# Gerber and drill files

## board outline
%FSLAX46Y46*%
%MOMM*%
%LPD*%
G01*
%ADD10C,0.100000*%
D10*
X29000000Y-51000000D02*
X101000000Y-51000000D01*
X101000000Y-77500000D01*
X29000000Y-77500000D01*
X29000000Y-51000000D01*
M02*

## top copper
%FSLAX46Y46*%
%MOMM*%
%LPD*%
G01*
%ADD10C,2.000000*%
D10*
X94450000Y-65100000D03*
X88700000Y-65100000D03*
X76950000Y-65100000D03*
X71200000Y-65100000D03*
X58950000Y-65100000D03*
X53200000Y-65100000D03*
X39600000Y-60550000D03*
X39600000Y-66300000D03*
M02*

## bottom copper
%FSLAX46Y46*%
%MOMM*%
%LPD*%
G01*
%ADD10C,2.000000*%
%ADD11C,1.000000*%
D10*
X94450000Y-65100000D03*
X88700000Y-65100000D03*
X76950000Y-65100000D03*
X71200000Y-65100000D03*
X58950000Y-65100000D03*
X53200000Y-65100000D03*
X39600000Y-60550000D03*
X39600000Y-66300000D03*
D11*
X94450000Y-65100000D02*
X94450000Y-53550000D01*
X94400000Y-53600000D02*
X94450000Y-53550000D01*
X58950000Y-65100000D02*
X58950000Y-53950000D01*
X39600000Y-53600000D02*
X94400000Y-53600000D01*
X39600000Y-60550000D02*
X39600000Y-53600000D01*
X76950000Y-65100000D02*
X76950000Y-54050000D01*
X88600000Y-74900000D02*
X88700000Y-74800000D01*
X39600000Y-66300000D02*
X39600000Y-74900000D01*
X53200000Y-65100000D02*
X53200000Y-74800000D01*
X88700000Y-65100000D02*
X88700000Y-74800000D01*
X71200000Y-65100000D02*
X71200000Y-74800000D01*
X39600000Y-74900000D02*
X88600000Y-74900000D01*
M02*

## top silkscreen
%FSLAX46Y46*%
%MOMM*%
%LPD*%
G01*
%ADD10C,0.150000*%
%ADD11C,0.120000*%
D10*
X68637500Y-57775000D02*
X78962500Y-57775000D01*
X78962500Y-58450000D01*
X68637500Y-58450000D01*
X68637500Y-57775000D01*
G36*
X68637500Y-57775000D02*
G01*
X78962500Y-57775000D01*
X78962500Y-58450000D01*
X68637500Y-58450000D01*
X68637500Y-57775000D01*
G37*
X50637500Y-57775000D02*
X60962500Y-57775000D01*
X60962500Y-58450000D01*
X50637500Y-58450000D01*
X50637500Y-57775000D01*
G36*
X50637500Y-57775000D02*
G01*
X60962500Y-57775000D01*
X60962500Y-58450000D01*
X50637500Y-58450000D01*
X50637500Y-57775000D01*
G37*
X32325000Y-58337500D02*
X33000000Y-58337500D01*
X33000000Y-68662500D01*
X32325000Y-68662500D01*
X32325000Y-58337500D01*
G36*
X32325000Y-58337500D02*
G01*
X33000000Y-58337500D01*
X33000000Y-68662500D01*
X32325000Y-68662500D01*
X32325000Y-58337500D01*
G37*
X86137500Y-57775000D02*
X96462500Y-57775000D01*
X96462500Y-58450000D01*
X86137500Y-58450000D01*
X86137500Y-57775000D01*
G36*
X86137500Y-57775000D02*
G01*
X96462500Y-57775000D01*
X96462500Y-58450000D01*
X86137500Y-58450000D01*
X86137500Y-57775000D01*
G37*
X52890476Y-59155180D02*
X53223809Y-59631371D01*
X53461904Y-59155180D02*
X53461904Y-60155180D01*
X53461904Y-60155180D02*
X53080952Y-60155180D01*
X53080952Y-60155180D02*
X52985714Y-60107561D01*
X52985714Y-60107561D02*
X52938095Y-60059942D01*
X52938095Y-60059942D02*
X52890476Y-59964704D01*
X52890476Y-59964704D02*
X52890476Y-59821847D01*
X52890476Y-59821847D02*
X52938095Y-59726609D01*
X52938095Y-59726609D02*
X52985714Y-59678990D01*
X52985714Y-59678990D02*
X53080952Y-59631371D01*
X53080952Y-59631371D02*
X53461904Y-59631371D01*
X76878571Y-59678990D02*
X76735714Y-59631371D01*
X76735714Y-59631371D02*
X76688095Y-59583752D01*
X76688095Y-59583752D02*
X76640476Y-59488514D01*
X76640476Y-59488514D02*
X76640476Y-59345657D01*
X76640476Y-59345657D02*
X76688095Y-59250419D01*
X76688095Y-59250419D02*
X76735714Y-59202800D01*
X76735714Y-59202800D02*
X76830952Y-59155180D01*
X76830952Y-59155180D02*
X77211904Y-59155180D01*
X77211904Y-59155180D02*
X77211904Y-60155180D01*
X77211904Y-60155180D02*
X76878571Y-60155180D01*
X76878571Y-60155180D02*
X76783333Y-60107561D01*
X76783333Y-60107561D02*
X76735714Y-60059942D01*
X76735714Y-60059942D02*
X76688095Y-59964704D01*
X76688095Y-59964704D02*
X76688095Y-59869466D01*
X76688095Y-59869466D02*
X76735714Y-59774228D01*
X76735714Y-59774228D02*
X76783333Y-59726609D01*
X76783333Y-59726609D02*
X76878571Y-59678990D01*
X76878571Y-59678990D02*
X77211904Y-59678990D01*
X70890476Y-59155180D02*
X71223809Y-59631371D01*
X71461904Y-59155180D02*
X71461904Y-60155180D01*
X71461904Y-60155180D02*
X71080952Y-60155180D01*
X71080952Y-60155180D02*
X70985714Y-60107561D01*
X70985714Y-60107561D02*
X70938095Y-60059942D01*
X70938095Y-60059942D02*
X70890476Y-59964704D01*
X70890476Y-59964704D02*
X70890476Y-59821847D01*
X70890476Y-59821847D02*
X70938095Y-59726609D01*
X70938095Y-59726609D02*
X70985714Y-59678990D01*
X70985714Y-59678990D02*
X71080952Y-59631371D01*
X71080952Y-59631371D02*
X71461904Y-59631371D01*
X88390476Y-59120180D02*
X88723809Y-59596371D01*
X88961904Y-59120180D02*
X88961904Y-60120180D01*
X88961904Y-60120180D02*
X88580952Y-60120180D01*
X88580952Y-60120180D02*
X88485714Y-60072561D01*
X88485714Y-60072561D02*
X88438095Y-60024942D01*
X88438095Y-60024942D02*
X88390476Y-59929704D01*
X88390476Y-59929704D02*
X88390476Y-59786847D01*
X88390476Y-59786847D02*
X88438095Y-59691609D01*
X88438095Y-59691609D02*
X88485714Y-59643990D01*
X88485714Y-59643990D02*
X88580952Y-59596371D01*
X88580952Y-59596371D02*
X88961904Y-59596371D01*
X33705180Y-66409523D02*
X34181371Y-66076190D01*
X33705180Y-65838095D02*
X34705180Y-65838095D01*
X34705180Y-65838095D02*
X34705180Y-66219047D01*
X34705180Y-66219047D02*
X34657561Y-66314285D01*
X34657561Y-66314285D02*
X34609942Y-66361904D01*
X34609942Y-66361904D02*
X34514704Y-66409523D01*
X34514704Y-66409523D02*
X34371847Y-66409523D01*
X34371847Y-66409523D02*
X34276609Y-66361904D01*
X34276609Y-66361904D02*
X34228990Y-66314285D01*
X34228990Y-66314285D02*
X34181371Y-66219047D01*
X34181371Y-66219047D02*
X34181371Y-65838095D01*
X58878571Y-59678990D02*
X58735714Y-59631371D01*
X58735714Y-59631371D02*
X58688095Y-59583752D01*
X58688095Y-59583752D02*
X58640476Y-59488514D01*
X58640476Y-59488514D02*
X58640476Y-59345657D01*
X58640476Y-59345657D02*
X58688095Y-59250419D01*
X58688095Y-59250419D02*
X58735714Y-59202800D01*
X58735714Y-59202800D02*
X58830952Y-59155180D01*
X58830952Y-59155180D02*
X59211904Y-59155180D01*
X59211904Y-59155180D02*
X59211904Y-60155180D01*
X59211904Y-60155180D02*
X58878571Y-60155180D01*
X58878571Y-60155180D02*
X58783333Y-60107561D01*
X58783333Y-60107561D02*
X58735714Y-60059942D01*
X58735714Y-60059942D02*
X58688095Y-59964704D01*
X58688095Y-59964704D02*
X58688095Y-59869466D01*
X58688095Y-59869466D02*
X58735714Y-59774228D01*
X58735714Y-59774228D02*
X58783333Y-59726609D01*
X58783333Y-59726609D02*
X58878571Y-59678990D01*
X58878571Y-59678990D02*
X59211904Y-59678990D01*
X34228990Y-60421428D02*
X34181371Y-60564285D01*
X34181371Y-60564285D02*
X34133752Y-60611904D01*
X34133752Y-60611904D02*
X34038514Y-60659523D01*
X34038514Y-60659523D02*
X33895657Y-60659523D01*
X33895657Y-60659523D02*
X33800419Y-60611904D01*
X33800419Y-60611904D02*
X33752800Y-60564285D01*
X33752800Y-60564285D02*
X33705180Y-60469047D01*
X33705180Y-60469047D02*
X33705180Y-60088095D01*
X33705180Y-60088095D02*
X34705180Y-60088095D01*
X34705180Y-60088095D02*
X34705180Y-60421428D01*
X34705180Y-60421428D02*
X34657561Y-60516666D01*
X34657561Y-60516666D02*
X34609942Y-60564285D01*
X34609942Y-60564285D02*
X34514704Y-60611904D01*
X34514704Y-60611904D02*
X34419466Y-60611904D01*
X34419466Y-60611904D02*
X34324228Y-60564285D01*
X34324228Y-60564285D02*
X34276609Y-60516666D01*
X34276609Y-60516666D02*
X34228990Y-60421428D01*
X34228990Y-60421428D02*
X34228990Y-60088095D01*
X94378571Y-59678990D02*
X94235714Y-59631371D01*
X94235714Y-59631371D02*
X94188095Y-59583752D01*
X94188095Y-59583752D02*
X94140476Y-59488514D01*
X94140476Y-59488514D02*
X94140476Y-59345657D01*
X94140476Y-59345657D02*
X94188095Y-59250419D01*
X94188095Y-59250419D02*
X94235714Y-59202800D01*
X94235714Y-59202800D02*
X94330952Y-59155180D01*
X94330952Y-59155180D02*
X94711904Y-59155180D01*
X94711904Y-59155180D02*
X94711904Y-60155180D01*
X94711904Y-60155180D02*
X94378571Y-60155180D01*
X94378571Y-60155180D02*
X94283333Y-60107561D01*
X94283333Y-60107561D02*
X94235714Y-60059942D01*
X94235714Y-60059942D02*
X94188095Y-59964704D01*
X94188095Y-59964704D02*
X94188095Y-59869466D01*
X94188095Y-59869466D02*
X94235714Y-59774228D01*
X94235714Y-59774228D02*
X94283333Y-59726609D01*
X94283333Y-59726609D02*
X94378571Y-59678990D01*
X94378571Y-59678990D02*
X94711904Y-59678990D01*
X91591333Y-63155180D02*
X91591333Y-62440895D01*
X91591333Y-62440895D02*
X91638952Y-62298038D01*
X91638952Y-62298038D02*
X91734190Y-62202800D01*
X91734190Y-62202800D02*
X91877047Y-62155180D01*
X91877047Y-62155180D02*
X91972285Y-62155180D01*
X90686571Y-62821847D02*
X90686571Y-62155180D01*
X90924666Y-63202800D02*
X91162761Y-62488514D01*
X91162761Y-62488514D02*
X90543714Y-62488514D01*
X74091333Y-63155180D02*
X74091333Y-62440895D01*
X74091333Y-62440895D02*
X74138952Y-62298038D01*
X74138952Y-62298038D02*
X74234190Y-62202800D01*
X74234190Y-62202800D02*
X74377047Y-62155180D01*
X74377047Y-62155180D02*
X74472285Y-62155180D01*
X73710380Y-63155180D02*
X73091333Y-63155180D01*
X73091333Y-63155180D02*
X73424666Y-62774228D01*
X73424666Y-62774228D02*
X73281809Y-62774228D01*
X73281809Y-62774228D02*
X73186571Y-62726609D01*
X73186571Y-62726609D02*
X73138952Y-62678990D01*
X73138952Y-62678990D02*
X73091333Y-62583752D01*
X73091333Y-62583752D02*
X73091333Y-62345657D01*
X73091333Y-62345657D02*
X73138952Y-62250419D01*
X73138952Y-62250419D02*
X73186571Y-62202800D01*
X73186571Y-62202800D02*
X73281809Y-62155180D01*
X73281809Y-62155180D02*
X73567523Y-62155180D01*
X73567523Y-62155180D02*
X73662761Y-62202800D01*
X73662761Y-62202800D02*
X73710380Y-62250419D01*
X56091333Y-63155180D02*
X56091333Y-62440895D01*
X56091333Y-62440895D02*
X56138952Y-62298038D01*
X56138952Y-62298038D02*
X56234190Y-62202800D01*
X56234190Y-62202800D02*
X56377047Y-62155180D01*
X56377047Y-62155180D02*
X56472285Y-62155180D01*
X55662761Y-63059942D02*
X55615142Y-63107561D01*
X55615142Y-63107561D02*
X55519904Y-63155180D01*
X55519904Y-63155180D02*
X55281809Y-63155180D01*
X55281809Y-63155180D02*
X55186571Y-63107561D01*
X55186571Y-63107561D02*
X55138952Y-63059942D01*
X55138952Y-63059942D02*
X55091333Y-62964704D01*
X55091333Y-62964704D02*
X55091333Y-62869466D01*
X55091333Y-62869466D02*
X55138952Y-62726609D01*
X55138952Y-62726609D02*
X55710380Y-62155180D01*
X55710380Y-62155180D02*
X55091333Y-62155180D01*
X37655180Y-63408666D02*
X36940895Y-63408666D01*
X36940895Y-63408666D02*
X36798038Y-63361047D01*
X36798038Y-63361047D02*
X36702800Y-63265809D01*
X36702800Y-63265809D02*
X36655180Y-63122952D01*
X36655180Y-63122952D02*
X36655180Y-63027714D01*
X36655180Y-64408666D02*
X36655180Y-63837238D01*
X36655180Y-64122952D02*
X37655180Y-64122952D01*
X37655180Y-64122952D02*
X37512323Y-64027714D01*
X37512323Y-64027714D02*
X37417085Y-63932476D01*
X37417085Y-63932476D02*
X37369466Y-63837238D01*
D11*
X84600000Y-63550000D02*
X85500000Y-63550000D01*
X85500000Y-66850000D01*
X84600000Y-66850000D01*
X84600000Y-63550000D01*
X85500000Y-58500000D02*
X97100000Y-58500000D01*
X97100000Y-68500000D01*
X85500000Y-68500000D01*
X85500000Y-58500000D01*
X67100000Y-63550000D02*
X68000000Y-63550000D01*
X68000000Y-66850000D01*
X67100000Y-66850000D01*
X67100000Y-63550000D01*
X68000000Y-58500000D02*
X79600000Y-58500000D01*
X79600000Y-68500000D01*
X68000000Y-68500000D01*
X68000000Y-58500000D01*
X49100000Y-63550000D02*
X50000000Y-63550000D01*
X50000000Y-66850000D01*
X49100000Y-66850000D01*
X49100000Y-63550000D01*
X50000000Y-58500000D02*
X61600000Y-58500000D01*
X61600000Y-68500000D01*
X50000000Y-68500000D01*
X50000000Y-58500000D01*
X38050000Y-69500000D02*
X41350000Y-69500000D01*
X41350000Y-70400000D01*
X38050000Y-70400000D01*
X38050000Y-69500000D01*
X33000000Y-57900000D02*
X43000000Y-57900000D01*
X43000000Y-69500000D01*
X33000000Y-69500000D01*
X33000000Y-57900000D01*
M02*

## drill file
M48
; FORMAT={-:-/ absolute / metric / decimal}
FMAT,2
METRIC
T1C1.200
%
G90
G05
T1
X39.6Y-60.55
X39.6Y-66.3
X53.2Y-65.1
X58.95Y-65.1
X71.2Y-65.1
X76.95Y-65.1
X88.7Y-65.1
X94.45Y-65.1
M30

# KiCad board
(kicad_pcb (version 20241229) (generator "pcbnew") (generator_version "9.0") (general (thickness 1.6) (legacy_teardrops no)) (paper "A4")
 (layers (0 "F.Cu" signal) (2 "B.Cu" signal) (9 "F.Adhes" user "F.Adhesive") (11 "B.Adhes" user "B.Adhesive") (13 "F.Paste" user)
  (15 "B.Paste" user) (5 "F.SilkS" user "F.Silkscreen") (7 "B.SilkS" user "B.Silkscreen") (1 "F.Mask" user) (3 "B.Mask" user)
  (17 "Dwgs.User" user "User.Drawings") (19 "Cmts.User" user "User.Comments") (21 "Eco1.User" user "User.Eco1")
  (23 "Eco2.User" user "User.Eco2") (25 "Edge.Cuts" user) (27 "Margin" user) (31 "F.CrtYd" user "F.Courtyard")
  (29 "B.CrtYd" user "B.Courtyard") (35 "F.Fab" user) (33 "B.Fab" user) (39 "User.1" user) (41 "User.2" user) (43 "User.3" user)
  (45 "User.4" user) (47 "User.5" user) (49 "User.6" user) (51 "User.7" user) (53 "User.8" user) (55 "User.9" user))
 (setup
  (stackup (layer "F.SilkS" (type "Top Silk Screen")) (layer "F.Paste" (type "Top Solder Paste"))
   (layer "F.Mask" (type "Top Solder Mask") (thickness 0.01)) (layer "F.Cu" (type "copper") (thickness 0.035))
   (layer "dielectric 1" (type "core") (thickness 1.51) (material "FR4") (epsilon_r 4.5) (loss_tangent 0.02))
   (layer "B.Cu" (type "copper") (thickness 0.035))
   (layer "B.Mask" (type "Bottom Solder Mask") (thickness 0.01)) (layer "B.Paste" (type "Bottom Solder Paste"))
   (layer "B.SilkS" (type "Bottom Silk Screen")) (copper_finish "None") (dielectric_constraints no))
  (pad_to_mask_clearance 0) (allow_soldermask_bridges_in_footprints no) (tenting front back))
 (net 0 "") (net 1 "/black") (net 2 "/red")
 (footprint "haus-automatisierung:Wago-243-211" (layer "F.Cu") (at 97.1 68.5 180)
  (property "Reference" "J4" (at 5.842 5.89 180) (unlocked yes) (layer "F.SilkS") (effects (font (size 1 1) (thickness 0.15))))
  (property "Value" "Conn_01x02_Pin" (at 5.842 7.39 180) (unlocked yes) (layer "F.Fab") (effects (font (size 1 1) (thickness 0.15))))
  (fp_rect (start 11.6 1.65) (end 12.5 4.95) (stroke (width 0.12) (type default)) (fill no) (layer "F.SilkS"))
  (fp_rect (start 0 0) (end 11.6 10) (stroke (width 0.12) (type default)) (fill no) (layer "F.SilkS"))
  (pad "1" thru_hole circle (at 2.65 3.4 180) (size 2 2) (drill 1.2) (layers "*.Cu" "*.Mask") (remove_unused_layers no) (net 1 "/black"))
  (pad "2" thru_hole circle (at 8.4 3.4 180) (size 2 2) (drill 1.2) (layers "*.Cu" "*.Mask") (remove_unused_layers no) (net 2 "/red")))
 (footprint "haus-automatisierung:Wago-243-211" (layer "F.Cu") (at 79.6 68.5 180)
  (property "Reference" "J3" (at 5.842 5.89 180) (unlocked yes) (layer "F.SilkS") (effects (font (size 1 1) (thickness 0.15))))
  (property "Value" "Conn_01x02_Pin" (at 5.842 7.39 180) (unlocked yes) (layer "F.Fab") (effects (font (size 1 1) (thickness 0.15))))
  (fp_rect (start 11.6 1.65) (end 12.5 4.95) (stroke (width 0.12) (type default)) (fill no) (layer "F.SilkS"))
  (fp_rect (start 0 0) (end 11.6 10) (stroke (width 0.12) (type default)) (fill no) (layer "F.SilkS"))
  (pad "1" thru_hole circle (at 2.65 3.4 180) (size 2 2) (drill 1.2) (layers "*.Cu" "*.Mask") (remove_unused_layers no) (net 1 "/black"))
  (pad "2" thru_hole circle (at 8.4 3.4 180) (size 2 2) (drill 1.2) (layers "*.Cu" "*.Mask") (remove_unused_layers no) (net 2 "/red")))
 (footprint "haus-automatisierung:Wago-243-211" (layer "F.Cu") (at 61.6 68.5 180)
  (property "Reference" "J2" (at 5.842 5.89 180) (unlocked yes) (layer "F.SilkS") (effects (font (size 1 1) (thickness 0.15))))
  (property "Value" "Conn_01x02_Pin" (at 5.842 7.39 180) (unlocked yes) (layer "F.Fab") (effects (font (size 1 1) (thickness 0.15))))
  (fp_rect (start 11.6 1.65) (end 12.5 4.95) (stroke (width 0.12) (type default)) (fill no) (layer "F.SilkS"))
  (fp_rect (start 0 0) (end 11.6 10) (stroke (width 0.12) (type default)) (fill no) (layer "F.SilkS"))
  (pad "1" thru_hole circle (at 2.65 3.4 180) (size 2 2) (drill 1.2) (layers "*.Cu" "*.Mask") (remove_unused_layers no) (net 1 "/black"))
  (pad "2" thru_hole circle (at 8.4 3.4 180) (size 2 2) (drill 1.2) (layers "*.Cu" "*.Mask") (remove_unused_layers no) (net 2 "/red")))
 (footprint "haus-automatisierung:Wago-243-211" (layer "F.Cu") (at 43 57.9 -90)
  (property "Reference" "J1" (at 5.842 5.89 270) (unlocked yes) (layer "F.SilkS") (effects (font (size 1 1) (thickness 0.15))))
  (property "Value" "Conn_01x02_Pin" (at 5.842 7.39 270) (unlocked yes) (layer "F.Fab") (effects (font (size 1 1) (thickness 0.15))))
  (fp_rect (start 11.6 1.65) (end 12.5 4.95) (stroke (width 0.12) (type default)) (fill no) (layer "F.SilkS"))
  (fp_rect (start 0 0) (end 11.6 10) (stroke (width 0.12) (type default)) (fill no) (layer "F.SilkS"))
  (pad "1" thru_hole circle (at 2.65 3.4 270) (size 2 2) (drill 1.2) (layers "*.Cu" "*.Mask") (remove_unused_layers no) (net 1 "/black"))
  (pad "2" thru_hole circle (at 8.4 3.4 270) (size 2 2) (drill 1.2) (layers "*.Cu" "*.Mask") (remove_unused_layers no) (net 2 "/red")))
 (gr_rect (start 68.6375 57.775) (end 78.9625 58.45) (stroke (width 0.15) (type solid)) (fill yes) (layer "F.SilkS"))
 (gr_rect (start 50.6375 57.775) (end 60.9625 58.45) (stroke (width 0.15) (type solid)) (fill yes) (layer "F.SilkS"))
 (gr_rect (start 32.325 58.3375) (end 33 68.6625) (stroke (width 0.15) (type solid)) (fill yes) (layer "F.SilkS"))
 (gr_rect (start 86.1375 57.775) (end 96.4625 58.45) (stroke (width 0.15) (type solid)) (fill yes) (layer "F.SilkS"))
 (gr_rect (start 29 51) (end 101 77.5) (stroke (width 0.1) (type default)) (fill no) (layer "Edge.Cuts"))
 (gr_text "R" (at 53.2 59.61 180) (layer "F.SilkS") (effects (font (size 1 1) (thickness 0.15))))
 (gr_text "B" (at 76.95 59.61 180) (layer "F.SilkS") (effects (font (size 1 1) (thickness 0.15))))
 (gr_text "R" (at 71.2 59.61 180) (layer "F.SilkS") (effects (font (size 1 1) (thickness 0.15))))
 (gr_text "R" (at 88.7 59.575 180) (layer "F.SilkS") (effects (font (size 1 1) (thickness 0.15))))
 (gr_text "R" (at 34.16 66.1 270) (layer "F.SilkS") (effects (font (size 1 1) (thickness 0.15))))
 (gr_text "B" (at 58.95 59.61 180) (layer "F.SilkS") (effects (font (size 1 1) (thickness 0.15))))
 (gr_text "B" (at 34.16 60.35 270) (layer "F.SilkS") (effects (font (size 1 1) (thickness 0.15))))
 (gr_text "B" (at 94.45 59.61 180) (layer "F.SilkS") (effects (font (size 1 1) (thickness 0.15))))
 (segment (start 94.45 65.1) (end 94.45 53.55) (width 1) (layer "B.Cu") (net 1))
 (segment (start 94.4 53.6) (end 94.45 53.55) (width 1) (layer "B.Cu") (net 1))
 (segment (start 58.95 65.1) (end 58.95 53.95) (width 1) (layer "B.Cu") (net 1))
 (segment (start 39.6 53.6) (end 94.4 53.6) (width 1) (layer "B.Cu") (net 1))
 (segment (start 39.6 60.55) (end 39.6 53.6) (width 1) (layer "B.Cu") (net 1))
 (segment (start 76.95 65.1) (end 76.95 54.05) (width 1) (layer "B.Cu") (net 1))
 (segment (start 88.6 74.9) (end 88.7 74.8) (width 1) (layer "B.Cu") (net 2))
 (segment (start 39.6 66.3) (end 39.6 74.9) (width 1) (layer "B.Cu") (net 2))
 (segment (start 53.2 65.1) (end 53.2 74.8) (width 1) (layer "B.Cu") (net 2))
 (segment (start 88.7 65.1) (end 88.7 74.8) (width 1) (layer "B.Cu") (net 2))
 (segment (start 71.2 65.1) (end 71.2 74.8) (width 1) (layer "B.Cu") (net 2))
 (segment (start 39.6 74.9) (end 88.6 74.9) (width 1) (layer "B.Cu") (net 2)))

